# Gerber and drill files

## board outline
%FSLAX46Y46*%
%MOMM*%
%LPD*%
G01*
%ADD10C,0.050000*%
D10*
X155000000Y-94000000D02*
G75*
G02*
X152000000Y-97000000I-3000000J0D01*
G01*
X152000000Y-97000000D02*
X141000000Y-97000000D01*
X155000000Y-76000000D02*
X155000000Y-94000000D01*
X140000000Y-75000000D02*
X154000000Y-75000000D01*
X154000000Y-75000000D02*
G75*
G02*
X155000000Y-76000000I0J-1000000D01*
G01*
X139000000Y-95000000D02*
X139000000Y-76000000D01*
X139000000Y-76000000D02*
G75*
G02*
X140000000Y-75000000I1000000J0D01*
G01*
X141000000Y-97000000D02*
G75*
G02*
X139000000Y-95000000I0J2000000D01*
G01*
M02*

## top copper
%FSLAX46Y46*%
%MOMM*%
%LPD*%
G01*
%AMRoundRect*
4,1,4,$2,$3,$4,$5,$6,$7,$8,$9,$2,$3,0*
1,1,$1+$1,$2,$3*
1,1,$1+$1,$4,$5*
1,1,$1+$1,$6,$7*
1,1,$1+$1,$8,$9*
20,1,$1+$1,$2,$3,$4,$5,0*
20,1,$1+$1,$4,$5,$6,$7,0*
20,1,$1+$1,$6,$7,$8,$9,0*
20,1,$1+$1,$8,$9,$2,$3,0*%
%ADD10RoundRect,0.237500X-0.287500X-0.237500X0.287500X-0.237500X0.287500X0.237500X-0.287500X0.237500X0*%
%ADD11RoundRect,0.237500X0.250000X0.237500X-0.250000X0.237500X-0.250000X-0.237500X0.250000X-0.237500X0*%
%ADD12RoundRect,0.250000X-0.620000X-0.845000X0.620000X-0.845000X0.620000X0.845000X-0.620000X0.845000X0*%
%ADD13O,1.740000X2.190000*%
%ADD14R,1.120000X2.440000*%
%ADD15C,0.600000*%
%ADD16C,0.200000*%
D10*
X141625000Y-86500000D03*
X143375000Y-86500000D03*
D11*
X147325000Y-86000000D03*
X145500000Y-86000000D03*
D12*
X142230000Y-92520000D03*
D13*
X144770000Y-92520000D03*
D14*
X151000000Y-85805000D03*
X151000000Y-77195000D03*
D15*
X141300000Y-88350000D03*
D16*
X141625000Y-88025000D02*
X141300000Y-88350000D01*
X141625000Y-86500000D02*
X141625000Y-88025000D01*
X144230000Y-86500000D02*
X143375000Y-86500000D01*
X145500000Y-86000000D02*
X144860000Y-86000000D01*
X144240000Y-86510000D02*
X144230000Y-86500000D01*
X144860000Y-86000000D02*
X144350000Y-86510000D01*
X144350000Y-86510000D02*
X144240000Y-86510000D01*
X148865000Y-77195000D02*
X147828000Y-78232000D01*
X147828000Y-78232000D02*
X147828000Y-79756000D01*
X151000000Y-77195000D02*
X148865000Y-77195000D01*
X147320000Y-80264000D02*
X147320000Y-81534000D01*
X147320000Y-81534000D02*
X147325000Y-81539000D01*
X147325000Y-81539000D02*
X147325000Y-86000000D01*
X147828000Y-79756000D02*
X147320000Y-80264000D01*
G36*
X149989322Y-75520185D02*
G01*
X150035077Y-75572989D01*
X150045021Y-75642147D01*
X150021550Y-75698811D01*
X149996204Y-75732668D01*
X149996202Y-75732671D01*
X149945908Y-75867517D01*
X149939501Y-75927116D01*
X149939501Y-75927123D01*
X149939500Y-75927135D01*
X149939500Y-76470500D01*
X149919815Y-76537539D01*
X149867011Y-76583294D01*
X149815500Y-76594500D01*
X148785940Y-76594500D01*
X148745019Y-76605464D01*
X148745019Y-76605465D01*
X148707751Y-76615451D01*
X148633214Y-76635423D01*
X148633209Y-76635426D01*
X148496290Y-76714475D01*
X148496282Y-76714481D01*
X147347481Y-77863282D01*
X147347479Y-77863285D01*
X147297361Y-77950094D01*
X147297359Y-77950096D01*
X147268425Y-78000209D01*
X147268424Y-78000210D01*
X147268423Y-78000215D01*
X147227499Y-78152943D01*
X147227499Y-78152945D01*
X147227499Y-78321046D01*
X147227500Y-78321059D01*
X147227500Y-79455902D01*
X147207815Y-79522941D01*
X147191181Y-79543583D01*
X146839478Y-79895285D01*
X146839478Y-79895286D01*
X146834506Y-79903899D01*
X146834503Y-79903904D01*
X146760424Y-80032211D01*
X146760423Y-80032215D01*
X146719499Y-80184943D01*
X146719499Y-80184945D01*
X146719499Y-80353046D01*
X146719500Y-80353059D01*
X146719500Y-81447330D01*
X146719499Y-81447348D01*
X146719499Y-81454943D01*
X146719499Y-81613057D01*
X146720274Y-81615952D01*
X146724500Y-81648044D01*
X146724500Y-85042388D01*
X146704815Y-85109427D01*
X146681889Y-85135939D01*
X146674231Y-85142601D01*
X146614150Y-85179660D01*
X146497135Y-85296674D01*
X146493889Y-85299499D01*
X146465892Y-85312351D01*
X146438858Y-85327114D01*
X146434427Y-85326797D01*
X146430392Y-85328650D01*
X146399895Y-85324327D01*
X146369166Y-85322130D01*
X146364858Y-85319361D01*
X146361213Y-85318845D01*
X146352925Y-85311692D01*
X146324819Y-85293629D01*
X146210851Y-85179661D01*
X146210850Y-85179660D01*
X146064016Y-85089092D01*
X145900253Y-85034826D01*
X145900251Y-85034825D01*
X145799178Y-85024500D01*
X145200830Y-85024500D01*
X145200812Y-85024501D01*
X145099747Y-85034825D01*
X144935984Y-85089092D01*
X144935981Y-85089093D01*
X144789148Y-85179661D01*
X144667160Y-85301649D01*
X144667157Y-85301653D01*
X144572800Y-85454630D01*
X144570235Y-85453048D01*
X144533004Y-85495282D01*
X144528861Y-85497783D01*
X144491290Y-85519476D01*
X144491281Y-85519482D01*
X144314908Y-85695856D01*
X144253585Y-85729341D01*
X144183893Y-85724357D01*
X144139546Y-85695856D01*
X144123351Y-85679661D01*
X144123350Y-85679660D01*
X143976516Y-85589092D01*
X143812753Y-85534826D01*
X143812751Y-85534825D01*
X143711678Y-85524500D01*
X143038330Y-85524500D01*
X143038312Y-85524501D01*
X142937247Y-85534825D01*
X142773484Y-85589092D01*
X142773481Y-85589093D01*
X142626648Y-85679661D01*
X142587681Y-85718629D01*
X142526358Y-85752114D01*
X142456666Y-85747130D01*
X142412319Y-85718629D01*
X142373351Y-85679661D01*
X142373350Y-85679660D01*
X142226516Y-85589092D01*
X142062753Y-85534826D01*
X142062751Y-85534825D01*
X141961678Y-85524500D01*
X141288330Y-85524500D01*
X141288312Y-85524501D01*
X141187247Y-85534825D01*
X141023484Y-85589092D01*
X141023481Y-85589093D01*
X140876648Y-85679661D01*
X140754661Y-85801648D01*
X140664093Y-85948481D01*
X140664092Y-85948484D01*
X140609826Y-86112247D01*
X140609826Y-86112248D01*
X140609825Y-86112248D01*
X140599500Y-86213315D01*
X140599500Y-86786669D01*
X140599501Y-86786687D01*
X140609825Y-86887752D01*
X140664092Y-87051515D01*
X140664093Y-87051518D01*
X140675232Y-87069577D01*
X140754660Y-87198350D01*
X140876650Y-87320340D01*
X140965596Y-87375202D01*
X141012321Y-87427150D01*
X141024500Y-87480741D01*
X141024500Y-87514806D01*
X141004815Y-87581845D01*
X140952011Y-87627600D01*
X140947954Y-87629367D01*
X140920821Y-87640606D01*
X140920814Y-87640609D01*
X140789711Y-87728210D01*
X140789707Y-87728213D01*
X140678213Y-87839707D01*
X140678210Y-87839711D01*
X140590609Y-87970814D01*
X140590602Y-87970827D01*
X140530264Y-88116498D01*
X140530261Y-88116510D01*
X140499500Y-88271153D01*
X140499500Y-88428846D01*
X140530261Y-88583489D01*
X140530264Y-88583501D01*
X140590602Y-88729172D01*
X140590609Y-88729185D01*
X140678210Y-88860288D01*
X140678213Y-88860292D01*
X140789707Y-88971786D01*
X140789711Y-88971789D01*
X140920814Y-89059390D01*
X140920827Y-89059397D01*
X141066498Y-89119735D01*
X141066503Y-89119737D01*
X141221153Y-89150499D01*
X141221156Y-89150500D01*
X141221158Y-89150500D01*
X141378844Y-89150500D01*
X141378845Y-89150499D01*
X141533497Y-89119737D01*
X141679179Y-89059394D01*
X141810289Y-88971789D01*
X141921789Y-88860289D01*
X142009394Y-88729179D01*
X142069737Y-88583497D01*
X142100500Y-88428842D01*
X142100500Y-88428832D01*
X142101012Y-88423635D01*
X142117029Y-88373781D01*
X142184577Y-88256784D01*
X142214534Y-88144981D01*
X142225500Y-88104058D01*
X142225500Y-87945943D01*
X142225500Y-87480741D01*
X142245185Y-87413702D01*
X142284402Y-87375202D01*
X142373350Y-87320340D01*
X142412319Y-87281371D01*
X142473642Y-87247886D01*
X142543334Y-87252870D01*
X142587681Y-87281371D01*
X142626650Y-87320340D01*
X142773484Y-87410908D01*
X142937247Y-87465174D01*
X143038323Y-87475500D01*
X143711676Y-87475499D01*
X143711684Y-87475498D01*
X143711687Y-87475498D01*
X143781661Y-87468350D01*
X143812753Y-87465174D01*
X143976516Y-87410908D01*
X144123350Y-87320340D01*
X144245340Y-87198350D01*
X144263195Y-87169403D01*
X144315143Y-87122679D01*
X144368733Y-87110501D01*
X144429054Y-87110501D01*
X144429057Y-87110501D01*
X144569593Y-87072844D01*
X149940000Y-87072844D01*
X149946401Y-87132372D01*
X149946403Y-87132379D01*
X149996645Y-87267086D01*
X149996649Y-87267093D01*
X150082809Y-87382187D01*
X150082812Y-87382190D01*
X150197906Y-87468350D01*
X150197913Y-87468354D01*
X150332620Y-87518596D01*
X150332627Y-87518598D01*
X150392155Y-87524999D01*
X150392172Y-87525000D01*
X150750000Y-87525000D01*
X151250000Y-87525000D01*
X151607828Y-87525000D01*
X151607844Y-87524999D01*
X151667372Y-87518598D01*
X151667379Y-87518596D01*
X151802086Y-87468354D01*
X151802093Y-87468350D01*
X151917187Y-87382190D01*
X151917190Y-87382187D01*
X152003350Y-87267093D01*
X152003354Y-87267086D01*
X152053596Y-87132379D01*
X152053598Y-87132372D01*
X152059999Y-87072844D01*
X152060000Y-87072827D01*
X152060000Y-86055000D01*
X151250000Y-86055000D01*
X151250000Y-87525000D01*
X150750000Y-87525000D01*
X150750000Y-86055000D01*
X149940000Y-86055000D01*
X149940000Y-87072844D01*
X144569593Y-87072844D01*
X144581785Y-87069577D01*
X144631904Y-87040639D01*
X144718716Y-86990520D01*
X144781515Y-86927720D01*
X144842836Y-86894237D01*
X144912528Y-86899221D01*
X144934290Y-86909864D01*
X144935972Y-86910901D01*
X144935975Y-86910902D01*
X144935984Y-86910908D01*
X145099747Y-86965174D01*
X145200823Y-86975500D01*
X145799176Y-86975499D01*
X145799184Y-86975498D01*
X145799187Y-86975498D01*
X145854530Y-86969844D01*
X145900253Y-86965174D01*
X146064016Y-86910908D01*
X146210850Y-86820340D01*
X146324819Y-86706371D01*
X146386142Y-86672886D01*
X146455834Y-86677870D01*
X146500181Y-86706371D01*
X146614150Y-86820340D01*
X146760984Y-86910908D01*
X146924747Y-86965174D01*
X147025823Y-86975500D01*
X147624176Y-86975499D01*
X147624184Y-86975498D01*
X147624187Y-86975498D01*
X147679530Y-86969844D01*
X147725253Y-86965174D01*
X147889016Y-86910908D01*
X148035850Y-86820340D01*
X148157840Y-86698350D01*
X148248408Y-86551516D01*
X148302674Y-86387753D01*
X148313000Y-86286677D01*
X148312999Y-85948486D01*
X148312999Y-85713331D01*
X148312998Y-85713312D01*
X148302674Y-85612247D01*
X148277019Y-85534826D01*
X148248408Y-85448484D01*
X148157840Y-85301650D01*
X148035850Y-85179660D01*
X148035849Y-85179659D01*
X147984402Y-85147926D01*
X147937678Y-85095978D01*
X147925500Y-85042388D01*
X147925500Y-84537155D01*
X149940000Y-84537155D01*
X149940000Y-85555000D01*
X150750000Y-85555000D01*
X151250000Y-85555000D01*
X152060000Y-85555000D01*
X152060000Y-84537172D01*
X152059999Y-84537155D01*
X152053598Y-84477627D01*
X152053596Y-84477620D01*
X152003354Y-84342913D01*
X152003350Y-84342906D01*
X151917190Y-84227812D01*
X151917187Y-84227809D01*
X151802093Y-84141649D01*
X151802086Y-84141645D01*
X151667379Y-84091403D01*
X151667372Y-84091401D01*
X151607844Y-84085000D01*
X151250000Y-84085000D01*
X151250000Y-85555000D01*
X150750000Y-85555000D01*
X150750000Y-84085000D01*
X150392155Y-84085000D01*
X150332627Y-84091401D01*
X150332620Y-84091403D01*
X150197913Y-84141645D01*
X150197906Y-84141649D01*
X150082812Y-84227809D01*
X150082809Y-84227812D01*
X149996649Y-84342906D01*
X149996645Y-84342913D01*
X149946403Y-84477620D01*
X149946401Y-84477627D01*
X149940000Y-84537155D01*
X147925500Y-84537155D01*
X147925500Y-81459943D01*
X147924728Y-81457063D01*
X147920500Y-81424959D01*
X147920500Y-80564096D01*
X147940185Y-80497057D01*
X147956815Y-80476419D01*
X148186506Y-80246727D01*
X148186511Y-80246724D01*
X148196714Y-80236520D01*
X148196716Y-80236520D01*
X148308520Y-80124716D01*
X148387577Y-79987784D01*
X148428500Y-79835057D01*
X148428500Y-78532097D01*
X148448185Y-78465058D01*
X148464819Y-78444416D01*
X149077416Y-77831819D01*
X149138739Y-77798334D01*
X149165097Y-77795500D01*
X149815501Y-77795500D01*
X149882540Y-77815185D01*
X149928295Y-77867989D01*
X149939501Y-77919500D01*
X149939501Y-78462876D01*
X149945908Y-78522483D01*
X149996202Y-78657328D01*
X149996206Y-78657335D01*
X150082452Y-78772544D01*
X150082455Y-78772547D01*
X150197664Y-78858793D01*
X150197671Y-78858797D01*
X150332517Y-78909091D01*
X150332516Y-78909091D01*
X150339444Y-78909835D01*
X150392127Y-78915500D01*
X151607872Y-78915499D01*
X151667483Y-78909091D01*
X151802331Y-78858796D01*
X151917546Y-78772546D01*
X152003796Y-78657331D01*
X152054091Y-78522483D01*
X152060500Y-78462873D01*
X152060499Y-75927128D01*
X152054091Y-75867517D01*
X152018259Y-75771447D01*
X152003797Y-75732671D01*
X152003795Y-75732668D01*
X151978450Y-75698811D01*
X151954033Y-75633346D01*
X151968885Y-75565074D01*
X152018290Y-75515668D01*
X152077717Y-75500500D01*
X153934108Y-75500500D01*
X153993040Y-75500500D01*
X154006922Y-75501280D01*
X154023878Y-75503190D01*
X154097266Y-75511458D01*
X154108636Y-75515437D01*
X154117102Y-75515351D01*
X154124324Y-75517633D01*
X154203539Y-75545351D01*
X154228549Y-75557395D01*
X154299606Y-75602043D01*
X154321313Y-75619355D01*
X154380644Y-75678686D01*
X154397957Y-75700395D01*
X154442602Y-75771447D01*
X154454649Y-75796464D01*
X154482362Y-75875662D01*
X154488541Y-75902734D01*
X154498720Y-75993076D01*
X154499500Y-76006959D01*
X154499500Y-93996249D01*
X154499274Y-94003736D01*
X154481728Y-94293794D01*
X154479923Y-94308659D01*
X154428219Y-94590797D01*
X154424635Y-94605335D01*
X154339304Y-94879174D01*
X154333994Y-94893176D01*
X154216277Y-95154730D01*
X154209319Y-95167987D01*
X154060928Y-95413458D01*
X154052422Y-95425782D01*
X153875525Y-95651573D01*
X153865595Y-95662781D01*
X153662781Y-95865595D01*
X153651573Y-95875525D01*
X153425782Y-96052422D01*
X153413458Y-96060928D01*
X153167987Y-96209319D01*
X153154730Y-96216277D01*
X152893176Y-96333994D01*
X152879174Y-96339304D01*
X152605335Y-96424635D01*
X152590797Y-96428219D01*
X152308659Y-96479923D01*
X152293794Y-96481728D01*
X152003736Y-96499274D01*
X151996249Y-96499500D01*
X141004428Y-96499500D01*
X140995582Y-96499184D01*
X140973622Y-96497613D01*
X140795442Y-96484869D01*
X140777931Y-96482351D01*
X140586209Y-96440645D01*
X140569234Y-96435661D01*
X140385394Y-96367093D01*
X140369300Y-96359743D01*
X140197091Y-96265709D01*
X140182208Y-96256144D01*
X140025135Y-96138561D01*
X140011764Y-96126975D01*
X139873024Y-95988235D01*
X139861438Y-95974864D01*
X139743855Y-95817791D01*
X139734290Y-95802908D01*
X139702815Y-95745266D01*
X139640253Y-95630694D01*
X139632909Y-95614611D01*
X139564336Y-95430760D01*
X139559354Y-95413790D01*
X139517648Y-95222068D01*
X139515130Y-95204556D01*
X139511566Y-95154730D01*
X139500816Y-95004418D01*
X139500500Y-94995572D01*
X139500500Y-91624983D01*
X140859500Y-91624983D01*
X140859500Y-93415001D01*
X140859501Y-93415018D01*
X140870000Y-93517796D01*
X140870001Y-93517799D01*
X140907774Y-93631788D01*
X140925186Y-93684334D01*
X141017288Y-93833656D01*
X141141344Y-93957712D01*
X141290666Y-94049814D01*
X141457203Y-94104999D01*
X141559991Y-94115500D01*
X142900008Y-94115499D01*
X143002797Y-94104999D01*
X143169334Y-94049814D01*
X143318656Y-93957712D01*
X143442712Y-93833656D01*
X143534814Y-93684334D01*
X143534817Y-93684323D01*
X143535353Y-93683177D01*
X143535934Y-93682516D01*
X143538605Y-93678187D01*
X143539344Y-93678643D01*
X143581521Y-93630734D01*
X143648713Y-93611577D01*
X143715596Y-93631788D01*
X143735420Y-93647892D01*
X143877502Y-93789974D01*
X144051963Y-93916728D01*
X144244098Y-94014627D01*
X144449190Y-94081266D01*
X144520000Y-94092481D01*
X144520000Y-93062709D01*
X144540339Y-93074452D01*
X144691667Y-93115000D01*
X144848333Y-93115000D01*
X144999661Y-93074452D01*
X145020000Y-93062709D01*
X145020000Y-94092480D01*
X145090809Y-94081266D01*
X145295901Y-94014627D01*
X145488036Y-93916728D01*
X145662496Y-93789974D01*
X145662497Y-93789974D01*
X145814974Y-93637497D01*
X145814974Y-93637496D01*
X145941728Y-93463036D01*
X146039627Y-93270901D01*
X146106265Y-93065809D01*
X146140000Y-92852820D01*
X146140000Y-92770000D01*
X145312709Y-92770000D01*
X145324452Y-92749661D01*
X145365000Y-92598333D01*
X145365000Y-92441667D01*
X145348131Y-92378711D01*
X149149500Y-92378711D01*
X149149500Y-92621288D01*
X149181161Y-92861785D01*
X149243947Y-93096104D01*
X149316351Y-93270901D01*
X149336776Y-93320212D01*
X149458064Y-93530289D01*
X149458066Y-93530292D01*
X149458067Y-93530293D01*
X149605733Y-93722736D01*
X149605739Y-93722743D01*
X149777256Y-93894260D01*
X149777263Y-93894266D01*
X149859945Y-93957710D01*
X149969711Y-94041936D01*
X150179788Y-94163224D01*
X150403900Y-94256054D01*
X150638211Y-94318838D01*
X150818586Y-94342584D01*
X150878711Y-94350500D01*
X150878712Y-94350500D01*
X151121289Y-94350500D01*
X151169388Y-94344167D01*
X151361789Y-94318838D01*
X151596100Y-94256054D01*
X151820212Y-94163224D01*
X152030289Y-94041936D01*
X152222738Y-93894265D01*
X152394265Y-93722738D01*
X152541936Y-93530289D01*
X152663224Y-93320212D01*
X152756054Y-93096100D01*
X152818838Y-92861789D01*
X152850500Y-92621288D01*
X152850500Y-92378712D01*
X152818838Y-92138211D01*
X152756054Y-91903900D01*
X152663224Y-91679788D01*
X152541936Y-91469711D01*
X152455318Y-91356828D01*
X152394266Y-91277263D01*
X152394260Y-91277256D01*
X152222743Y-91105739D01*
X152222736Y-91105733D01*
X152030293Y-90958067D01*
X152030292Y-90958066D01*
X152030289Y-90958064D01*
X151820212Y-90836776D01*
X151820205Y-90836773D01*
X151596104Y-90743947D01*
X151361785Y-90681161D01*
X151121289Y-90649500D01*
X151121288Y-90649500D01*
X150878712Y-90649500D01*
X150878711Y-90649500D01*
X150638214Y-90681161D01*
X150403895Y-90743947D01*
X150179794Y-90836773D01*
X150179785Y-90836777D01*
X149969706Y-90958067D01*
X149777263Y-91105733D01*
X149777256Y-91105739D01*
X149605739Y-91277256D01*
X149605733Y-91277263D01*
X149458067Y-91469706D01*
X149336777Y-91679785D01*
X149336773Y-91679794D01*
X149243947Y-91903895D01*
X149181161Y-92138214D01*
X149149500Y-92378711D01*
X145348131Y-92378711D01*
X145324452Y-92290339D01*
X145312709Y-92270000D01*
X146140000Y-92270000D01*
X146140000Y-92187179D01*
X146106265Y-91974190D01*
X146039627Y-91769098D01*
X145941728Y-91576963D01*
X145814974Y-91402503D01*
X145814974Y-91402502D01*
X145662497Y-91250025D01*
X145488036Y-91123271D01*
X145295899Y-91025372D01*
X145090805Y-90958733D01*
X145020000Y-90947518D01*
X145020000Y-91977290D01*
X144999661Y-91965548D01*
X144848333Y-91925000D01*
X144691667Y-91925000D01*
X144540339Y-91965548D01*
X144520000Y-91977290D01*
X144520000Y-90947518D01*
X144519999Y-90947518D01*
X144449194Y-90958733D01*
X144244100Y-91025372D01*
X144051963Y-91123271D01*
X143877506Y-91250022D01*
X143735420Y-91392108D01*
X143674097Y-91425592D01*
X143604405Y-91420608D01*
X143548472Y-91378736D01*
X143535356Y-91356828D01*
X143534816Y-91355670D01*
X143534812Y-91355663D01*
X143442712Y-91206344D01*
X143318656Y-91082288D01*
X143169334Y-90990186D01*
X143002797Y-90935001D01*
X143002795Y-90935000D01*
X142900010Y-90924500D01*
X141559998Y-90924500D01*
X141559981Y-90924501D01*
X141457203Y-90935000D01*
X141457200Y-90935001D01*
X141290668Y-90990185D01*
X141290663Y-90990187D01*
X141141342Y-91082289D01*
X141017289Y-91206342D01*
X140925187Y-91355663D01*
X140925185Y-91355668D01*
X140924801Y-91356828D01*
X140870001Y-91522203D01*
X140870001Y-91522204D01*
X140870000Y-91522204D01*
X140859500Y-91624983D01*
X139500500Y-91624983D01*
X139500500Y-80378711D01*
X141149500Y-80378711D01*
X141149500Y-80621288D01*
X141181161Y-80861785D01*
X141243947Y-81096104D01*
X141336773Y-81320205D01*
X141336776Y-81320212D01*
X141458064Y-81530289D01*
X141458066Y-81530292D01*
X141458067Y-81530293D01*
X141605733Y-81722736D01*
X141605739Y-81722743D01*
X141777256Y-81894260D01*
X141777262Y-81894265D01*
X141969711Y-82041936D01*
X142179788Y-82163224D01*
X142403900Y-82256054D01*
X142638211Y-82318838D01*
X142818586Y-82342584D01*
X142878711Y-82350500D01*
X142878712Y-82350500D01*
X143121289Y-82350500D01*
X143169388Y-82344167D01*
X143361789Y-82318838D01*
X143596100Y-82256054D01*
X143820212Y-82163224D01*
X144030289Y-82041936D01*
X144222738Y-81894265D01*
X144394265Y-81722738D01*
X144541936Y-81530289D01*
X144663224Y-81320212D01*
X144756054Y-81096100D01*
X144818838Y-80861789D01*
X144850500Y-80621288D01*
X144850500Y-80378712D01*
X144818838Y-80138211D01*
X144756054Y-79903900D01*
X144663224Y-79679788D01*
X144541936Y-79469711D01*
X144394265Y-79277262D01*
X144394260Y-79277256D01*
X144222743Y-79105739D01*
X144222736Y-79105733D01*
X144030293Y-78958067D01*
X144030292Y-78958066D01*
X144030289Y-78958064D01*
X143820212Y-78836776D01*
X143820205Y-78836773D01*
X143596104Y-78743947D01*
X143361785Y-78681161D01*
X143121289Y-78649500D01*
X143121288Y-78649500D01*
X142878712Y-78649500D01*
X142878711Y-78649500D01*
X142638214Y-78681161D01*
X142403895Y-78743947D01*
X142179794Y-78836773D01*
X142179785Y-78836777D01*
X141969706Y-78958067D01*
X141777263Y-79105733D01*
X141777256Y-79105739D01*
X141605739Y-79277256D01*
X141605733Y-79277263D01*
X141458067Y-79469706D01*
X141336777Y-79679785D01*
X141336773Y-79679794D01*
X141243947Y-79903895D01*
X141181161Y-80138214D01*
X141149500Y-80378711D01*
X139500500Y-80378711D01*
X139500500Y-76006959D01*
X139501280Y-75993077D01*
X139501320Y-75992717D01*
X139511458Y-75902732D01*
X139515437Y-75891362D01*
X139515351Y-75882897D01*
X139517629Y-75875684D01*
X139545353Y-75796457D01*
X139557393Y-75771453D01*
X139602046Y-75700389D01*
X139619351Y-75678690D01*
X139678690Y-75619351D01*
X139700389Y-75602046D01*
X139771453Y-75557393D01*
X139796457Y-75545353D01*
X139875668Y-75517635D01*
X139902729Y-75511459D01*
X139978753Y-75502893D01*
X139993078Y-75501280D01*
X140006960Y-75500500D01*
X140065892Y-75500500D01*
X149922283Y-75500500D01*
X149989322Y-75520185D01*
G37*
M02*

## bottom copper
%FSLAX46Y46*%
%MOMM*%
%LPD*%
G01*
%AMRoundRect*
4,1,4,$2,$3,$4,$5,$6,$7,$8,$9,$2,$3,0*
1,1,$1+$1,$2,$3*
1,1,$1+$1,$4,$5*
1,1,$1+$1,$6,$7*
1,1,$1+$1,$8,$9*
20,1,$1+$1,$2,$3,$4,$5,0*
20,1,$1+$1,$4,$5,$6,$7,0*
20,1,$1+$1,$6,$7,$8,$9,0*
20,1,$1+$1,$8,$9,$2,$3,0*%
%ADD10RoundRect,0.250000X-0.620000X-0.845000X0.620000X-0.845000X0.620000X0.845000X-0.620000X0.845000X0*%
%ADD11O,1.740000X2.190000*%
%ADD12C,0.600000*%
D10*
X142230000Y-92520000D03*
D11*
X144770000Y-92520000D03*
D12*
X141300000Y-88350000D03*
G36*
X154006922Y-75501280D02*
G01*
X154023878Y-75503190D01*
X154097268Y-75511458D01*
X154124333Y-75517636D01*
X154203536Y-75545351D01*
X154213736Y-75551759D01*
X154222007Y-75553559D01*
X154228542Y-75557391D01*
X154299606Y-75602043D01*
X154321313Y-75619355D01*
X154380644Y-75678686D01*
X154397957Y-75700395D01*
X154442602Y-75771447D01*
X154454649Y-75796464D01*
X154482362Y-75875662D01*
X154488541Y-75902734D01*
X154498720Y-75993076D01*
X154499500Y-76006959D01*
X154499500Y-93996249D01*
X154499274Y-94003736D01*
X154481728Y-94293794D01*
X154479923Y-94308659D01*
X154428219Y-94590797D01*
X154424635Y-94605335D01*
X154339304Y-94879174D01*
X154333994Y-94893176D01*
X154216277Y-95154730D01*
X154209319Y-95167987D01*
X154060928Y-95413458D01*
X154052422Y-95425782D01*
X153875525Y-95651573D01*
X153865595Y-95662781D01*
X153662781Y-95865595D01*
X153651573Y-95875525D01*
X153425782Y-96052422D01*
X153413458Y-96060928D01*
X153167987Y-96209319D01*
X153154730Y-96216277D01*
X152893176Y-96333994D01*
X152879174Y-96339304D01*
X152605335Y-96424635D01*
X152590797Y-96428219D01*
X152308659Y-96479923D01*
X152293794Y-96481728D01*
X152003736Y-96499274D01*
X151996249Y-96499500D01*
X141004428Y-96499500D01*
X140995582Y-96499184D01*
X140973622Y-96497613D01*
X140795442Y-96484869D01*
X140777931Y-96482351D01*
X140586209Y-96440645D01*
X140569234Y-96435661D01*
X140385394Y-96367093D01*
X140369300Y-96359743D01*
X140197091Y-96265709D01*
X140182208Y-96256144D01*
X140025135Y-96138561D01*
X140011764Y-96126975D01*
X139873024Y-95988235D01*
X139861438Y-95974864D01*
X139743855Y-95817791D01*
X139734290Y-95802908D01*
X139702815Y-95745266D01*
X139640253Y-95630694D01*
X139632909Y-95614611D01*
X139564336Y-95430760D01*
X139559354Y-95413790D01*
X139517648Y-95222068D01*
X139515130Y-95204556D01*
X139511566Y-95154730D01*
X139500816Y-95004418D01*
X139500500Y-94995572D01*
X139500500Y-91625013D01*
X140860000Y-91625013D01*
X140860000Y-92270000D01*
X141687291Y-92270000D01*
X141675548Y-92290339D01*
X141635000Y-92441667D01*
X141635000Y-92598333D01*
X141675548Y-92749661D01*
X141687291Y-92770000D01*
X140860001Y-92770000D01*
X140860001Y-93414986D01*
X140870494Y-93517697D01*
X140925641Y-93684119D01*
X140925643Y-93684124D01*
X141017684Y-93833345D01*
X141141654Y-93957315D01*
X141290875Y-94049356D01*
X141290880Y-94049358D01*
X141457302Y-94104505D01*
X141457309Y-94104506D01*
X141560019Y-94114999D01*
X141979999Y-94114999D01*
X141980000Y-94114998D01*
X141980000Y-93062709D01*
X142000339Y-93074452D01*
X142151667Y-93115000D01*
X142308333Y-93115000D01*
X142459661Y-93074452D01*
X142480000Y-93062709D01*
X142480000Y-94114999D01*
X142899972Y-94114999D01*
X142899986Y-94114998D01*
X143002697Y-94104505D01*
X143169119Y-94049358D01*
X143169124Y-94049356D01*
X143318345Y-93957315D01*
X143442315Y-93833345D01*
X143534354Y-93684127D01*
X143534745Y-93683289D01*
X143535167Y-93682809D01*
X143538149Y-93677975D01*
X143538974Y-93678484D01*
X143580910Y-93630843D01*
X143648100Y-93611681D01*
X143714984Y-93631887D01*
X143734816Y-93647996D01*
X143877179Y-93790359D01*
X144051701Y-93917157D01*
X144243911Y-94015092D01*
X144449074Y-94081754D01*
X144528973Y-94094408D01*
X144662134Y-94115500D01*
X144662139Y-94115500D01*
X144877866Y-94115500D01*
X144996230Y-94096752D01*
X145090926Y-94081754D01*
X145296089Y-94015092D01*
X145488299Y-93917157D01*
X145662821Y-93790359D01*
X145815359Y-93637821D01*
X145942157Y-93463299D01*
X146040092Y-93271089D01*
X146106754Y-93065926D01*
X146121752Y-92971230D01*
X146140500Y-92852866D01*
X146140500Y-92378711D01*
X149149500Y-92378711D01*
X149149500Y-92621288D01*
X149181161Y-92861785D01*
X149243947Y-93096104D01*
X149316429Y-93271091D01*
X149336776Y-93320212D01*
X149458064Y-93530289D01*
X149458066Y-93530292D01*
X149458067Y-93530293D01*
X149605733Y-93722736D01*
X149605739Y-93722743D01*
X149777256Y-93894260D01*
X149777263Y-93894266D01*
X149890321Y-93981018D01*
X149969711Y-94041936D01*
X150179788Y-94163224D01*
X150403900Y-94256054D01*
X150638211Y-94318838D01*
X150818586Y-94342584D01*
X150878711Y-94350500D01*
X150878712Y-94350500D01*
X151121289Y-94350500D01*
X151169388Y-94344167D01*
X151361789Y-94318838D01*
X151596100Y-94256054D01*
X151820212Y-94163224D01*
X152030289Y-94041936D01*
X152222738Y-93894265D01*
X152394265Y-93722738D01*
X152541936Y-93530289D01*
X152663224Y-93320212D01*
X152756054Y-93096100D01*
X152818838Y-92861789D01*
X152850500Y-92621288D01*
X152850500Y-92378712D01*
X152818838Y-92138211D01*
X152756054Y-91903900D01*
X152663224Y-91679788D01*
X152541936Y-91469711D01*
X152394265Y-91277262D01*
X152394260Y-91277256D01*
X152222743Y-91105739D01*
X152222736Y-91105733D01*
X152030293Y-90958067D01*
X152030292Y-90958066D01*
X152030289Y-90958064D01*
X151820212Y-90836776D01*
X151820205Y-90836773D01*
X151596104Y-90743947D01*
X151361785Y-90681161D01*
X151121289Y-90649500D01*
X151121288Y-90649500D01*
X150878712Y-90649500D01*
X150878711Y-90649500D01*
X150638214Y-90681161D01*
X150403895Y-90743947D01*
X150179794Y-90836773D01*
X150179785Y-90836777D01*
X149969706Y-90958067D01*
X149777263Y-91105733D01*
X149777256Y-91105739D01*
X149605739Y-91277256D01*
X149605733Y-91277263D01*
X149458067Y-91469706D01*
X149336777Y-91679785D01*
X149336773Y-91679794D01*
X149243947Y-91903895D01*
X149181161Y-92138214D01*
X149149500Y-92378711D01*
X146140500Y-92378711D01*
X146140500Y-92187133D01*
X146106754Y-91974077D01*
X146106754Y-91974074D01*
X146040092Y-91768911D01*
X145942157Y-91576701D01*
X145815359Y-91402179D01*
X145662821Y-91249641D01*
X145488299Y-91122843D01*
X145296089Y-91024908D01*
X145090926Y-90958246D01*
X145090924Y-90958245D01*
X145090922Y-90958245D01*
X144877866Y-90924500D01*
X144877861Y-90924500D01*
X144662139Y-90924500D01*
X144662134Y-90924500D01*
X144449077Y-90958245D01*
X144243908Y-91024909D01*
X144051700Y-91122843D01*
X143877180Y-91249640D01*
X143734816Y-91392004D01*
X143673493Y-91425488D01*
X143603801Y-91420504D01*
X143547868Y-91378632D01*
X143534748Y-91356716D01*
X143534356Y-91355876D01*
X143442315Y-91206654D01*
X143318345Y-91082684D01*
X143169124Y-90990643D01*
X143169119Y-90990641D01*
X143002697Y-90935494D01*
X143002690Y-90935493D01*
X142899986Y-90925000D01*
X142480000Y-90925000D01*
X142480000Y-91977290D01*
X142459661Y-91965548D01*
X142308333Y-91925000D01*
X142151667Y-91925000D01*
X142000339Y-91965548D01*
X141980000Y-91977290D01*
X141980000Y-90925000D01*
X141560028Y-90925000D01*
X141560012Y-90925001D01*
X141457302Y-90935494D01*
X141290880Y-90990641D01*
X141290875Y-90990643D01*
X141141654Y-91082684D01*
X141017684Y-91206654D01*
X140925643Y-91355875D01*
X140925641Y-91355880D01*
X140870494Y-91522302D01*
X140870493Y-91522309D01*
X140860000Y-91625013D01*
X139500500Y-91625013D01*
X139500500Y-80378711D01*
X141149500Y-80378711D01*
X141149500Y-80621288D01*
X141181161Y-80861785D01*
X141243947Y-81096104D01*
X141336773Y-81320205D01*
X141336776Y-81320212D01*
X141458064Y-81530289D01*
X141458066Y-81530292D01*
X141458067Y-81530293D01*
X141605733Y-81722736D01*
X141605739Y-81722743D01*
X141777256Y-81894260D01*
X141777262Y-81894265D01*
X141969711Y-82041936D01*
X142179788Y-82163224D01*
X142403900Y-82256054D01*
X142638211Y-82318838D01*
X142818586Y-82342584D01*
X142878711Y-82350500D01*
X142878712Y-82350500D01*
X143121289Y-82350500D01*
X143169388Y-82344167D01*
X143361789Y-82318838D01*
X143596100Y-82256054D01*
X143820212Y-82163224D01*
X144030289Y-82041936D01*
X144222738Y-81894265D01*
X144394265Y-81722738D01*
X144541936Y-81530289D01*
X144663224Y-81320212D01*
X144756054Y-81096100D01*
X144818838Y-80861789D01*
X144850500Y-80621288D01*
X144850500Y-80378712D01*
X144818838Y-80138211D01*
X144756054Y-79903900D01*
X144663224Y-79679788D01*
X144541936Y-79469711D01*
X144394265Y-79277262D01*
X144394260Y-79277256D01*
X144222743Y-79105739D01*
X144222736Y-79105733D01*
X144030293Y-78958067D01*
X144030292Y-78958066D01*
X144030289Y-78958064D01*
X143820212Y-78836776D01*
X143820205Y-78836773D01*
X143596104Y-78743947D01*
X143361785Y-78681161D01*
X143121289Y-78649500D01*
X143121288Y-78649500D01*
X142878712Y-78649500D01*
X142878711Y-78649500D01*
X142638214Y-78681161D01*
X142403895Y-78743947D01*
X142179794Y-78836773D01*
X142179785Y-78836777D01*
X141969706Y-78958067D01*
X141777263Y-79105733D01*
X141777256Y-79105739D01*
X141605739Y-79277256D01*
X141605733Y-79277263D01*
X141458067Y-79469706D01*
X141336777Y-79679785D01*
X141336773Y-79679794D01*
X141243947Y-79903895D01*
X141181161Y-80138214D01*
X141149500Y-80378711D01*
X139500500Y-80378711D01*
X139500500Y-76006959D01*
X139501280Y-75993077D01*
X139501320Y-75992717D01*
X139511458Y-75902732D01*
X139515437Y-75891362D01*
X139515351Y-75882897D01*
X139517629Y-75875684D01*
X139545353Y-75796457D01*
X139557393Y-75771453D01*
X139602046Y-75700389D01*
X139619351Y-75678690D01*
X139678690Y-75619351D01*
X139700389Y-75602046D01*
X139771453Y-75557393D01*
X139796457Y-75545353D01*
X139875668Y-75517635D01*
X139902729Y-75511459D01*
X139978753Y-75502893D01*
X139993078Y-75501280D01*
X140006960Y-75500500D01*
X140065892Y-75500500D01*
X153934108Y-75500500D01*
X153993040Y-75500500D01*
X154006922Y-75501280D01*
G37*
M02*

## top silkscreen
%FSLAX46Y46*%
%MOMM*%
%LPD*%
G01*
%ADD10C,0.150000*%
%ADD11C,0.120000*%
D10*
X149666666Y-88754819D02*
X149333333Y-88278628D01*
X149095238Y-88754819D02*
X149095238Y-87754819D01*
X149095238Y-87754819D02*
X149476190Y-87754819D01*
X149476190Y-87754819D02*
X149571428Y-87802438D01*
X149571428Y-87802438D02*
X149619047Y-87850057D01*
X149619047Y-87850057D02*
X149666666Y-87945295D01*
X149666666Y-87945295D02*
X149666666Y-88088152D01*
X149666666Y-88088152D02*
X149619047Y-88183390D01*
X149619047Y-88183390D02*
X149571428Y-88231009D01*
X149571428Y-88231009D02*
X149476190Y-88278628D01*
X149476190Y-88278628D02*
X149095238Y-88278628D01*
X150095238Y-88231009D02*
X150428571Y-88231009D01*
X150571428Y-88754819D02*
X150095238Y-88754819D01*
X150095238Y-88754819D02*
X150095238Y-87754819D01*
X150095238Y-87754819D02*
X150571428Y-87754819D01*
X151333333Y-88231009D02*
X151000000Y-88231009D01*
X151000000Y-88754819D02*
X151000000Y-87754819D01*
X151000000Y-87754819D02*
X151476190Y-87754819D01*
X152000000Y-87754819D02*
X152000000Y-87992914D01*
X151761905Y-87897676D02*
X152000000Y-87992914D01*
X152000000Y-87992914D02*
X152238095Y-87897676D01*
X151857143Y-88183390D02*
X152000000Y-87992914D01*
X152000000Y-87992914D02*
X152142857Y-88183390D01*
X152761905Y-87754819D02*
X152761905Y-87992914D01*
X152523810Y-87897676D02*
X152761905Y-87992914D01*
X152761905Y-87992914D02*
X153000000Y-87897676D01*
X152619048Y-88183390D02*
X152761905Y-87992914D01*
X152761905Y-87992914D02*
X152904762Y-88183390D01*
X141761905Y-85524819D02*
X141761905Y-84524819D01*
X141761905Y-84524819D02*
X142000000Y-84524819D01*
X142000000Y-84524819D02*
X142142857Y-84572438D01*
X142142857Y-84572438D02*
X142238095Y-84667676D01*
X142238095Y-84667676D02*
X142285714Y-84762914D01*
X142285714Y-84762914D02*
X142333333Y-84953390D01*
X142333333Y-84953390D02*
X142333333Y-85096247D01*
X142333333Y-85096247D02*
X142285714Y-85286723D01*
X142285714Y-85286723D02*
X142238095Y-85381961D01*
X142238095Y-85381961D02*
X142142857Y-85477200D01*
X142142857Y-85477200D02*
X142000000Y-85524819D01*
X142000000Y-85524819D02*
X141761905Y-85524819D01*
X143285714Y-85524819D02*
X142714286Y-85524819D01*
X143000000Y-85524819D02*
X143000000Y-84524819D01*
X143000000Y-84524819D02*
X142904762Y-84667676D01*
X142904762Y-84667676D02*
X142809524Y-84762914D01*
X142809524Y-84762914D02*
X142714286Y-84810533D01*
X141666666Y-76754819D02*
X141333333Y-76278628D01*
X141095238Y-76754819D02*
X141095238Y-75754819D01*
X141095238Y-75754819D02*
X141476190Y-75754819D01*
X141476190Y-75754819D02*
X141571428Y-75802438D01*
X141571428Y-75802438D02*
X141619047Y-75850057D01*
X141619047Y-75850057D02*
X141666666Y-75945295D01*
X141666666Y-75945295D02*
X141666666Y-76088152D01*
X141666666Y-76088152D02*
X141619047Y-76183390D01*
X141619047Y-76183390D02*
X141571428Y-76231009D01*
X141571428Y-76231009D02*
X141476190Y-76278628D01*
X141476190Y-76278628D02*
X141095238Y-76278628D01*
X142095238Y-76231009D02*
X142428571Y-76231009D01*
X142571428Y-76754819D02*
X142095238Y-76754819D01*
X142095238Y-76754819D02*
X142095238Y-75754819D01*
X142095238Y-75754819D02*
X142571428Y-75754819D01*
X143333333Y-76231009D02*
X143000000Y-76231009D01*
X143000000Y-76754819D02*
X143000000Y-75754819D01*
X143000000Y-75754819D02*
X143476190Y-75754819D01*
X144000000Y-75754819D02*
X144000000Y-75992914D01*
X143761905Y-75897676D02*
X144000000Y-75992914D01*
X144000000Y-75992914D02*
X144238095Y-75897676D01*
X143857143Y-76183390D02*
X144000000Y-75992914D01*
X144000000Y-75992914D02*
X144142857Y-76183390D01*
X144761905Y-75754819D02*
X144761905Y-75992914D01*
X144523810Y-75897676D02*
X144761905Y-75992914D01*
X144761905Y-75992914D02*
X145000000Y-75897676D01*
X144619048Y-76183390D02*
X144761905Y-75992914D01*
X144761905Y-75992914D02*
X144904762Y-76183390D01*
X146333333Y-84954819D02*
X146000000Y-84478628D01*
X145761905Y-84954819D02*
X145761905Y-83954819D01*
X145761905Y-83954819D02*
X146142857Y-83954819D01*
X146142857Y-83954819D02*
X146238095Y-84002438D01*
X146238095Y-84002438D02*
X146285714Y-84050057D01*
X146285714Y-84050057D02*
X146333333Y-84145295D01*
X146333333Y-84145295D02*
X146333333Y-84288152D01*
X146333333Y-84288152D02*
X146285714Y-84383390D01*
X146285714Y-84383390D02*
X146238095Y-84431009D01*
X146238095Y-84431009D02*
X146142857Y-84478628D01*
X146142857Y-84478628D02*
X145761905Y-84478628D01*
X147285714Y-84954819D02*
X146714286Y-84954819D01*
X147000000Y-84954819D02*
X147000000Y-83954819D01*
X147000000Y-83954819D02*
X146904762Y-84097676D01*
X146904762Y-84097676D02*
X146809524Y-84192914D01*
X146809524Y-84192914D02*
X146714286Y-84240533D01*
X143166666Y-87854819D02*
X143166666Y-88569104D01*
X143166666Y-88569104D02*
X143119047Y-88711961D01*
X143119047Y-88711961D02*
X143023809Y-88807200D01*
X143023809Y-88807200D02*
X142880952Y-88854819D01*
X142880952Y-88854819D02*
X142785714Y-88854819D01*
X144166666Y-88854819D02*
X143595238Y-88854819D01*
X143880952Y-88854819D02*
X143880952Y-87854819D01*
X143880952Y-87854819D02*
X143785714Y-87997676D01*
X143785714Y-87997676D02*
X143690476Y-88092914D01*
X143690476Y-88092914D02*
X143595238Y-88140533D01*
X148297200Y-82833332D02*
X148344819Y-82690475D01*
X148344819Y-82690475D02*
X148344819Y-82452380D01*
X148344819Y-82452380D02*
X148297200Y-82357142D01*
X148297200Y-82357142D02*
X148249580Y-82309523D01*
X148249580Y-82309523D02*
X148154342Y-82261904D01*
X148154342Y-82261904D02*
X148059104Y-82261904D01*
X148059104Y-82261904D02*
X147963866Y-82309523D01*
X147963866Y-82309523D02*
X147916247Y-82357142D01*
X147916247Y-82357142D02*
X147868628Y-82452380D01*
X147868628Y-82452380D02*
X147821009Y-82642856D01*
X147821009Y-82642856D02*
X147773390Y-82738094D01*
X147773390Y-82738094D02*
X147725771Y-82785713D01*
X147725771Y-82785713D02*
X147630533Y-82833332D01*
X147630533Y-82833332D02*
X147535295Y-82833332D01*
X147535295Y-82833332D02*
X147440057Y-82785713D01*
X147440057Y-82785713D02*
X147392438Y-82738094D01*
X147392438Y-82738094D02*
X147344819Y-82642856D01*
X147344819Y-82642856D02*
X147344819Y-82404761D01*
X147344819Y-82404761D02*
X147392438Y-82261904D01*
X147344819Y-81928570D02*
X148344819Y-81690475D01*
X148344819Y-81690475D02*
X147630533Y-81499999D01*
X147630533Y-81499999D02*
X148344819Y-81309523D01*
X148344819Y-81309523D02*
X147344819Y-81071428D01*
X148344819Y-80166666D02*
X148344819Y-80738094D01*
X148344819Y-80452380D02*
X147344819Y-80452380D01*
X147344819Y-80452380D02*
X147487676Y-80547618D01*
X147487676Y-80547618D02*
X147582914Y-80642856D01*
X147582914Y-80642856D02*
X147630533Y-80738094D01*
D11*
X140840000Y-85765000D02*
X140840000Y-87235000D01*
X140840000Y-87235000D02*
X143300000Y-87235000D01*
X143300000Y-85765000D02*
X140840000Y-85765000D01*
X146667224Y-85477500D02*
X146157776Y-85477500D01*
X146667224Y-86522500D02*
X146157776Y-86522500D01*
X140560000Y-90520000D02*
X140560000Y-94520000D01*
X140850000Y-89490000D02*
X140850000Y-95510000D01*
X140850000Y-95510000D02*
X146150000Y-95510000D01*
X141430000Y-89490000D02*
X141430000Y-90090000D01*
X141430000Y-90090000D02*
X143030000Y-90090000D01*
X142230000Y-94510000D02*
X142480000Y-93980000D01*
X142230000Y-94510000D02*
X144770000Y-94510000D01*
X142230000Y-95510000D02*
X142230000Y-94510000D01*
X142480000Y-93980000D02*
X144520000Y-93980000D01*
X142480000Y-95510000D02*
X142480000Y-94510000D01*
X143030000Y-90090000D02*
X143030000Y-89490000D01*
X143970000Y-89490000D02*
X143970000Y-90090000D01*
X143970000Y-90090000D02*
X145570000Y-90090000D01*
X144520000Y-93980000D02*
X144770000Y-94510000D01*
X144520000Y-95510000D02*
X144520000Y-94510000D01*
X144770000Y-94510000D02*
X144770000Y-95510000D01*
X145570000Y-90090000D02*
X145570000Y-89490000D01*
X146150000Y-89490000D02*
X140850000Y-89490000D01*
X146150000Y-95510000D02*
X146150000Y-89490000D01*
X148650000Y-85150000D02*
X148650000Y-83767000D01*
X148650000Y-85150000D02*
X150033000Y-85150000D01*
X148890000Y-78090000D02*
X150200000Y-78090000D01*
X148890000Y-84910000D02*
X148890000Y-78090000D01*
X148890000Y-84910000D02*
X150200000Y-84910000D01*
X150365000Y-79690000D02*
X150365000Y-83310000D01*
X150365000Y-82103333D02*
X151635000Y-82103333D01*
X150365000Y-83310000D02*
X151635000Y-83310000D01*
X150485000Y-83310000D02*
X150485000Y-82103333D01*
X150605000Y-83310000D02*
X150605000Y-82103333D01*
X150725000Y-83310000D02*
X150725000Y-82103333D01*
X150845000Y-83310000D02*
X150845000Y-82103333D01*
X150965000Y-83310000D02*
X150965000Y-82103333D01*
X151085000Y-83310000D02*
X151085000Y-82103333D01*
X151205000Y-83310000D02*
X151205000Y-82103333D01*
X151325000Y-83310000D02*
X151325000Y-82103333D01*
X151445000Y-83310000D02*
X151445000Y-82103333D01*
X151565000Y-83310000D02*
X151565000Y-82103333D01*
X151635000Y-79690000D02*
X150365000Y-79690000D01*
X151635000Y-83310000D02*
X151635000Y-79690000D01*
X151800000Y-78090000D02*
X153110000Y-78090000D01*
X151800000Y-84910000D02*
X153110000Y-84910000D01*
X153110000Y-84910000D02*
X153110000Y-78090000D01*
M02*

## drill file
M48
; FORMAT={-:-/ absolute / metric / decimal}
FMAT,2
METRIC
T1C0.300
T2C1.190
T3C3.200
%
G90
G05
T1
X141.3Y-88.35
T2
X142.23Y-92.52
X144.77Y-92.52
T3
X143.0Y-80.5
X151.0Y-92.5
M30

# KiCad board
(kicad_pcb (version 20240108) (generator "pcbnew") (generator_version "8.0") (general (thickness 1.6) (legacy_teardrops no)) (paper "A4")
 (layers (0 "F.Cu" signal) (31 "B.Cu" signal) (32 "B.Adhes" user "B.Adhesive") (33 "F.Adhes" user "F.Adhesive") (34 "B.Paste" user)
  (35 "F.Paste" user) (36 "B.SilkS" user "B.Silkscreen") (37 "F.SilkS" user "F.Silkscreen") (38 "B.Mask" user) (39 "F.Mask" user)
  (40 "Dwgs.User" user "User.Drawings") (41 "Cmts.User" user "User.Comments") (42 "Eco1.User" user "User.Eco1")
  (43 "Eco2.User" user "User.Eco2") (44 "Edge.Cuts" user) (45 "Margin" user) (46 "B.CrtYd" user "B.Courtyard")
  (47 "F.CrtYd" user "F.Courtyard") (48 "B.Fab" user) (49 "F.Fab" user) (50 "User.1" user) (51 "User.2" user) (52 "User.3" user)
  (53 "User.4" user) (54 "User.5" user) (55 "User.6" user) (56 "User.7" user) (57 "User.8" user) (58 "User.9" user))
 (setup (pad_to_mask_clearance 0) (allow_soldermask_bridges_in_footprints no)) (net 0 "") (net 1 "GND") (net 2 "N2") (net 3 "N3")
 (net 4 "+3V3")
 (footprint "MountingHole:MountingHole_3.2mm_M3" (layer "F.Cu") (at 151 92.5)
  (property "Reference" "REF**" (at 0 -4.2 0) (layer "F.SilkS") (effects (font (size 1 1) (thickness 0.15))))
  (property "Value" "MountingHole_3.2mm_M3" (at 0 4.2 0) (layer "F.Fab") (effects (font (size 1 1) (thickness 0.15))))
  (pad "" np_thru_hole circle (at 0 0) (size 3.2 3.2) (drill 3.2) (layers "*.Cu" "*.Mask")))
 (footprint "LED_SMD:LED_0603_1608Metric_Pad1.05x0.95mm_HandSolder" (layer "F.Cu") (at 142.5 86.5)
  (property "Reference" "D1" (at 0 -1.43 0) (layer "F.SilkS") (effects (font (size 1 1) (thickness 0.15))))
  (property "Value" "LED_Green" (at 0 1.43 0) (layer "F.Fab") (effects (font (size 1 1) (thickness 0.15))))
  (fp_line (start -1.66 -0.735) (end -1.66 0.735) (stroke (width 0.12) (type solid)) (layer "F.SilkS"))
  (fp_line (start -1.66 0.735) (end 0.8 0.735) (stroke (width 0.12) (type solid)) (layer "F.SilkS"))
  (fp_line (start 0.8 -0.735) (end -1.66 -0.735) (stroke (width 0.12) (type solid)) (layer "F.SilkS"))
  (pad "1" smd roundrect (at -0.875 0) (size 1.05 0.95) (layers "F.Cu" "F.Paste" "F.Mask") (roundrect_rratio 0.25) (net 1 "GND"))
  (pad "2" smd roundrect (at 0.875 0) (size 1.05 0.95) (layers "F.Cu" "F.Paste" "F.Mask") (roundrect_rratio 0.25) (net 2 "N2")))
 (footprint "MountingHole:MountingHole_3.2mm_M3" (layer "F.Cu") (at 143 80.5)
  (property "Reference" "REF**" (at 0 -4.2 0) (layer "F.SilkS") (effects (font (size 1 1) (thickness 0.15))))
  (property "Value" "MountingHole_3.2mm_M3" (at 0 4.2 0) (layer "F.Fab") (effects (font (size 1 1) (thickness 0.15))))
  (pad "" np_thru_hole circle (at 0 0) (size 3.2 3.2) (drill 3.2) (layers "*.Cu" "*.Mask")))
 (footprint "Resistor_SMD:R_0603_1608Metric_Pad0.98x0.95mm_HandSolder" (layer "F.Cu") (at 146.4125 86 180)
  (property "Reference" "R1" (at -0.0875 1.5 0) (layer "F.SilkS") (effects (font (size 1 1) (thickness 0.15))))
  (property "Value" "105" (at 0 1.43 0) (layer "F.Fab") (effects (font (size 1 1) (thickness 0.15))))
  (fp_line (start -0.254724 0.5225) (end 0.254724 0.5225) (stroke (width 0.12) (type solid)) (layer "F.SilkS"))
  (fp_line (start -0.254724 -0.5225) (end 0.254724 -0.5225) (stroke (width 0.12) (type solid)) (layer "F.SilkS"))
  (pad "1" smd roundrect (at -0.9125 0 180) (size 0.975 0.95) (layers "F.Cu" "F.Paste" "F.Mask") (roundrect_rratio 0.25) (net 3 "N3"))
  (pad "2" smd roundrect (at 0.9125 0 180) (size 0.975 0.95) (layers "F.Cu" "F.Paste" "F.Mask") (roundrect_rratio 0.25) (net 2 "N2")))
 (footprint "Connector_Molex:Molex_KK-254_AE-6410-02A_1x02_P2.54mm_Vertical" (layer "F.Cu") (at 142.23 92.52)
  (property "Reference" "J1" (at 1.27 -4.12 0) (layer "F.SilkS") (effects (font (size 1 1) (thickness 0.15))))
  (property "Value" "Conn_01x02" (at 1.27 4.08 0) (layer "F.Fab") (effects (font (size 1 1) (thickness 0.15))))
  (fp_line (start -1.67 -2) (end -1.67 2) (stroke (width 0.12) (type solid)) (layer "F.SilkS"))
  (fp_line (start -1.38 -3.03) (end -1.38 2.99) (stroke (width 0.12) (type solid)) (layer "F.SilkS"))
  (fp_line (start -1.38 2.99) (end 3.92 2.99) (stroke (width 0.12) (type solid)) (layer "F.SilkS"))
  (fp_line (start -0.8 -3.03) (end -0.8 -2.43) (stroke (width 0.12) (type solid)) (layer "F.SilkS"))
  (fp_line (start -0.8 -2.43) (end 0.8 -2.43) (stroke (width 0.12) (type solid)) (layer "F.SilkS"))
  (fp_line (start 0 1.99) (end 0.25 1.46) (stroke (width 0.12) (type solid)) (layer "F.SilkS"))
  (fp_line (start 0 1.99) (end 2.54 1.99) (stroke (width 0.12) (type solid)) (layer "F.SilkS"))
  (fp_line (start 0 2.99) (end 0 1.99) (stroke (width 0.12) (type solid)) (layer "F.SilkS"))
  (fp_line (start 0.25 1.46) (end 2.29 1.46) (stroke (width 0.12) (type solid)) (layer "F.SilkS"))
  (fp_line (start 0.25 2.99) (end 0.25 1.99) (stroke (width 0.12) (type solid)) (layer "F.SilkS"))
  (fp_line (start 0.8 -2.43) (end 0.8 -3.03) (stroke (width 0.12) (type solid)) (layer "F.SilkS"))
  (fp_line (start 1.74 -3.03) (end 1.74 -2.43) (stroke (width 0.12) (type solid)) (layer "F.SilkS"))
  (fp_line (start 1.74 -2.43) (end 3.34 -2.43) (stroke (width 0.12) (type solid)) (layer "F.SilkS"))
  (fp_line (start 2.29 1.46) (end 2.54 1.99) (stroke (width 0.12) (type solid)) (layer "F.SilkS"))
  (fp_line (start 2.29 2.99) (end 2.29 1.99) (stroke (width 0.12) (type solid)) (layer "F.SilkS"))
  (fp_line (start 2.54 1.99) (end 2.54 2.99) (stroke (width 0.12) (type solid)) (layer "F.SilkS"))
  (fp_line (start 3.34 -2.43) (end 3.34 -3.03) (stroke (width 0.12) (type solid)) (layer "F.SilkS"))
  (fp_line (start 3.92 -3.03) (end -1.38 -3.03) (stroke (width 0.12) (type solid)) (layer "F.SilkS"))
  (fp_line (start 3.92 2.99) (end 3.92 -3.03) (stroke (width 0.12) (type solid)) (layer "F.SilkS"))
  (pad "1" thru_hole roundrect (at 0 0) (size 1.74 2.19) (drill 1.19) (layers "*.Cu" "*.Mask") (remove_unused_layers no)
   (roundrect_rratio 0.143678) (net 1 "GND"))
  (pad "2" thru_hole oval (at 2.54 0) (size 1.74 2.19) (drill 1.19) (layers "*.Cu" "*.Mask") (remove_unused_layers no) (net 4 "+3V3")))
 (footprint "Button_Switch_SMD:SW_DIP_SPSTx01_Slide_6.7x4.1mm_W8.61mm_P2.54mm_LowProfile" (layer "F.Cu") (at 151 81.5 90)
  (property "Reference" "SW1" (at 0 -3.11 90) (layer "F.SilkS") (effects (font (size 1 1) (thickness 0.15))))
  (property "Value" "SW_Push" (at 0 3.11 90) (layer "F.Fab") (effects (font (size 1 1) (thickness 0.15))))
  (fp_line (start -3.65 -2.35) (end -2.267 -2.35) (stroke (width 0.12) (type solid)) (layer "F.SilkS"))
  (fp_line (start -3.65 -2.35) (end -3.65 -0.967) (stroke (width 0.12) (type solid)) (layer "F.SilkS"))
  (fp_line (start 3.41 -2.11) (end 3.41 -0.8) (stroke (width 0.12) (type solid)) (layer "F.SilkS"))
  (fp_line (start -3.41 -2.11) (end 3.41 -2.11) (stroke (width 0.12) (type solid)) (layer "F.SilkS"))
  (fp_line (start -3.41 -2.11) (end -3.41 -0.8) (stroke (width 0.12) (type solid)) (layer "F.SilkS"))
  (fp_line (start 1.81 -0.635) (end -1.81 -0.635) (stroke (width 0.12) (type solid)) (layer "F.SilkS"))
  (fp_line (start -0.603333 -0.635) (end -0.603333 0.635) (stroke (width 0.12) (type solid)) (layer "F.SilkS"))
  (fp_line (start -1.81 -0.635) (end -1.81 0.635) (stroke (width 0.12) (type solid)) (layer "F.SilkS"))
  (fp_line (start -1.81 -0.515) (end -0.603333 -0.515) (stroke (width 0.12) (type solid)) (layer "F.SilkS"))
  (fp_line (start -1.81 -0.395) (end -0.603333 -0.395) (stroke (width 0.12) (type solid)) (layer "F.SilkS"))
  (fp_line (start -1.81 -0.275) (end -0.603333 -0.275) (stroke (width 0.12) (type solid)) (layer "F.SilkS"))
  (fp_line (start -1.81 -0.155) (end -0.603333 -0.155) (stroke (width 0.12) (type solid)) (layer "F.SilkS"))
  (fp_line (start -1.81 -0.035) (end -0.603333 -0.035) (stroke (width 0.12) (type solid)) (layer "F.SilkS"))
  (fp_line (start -1.81 0.085) (end -0.603333 0.085) (stroke (width 0.12) (type solid)) (layer "F.SilkS"))
  (fp_line (start -1.81 0.205) (end -0.603333 0.205) (stroke (width 0.12) (type solid)) (layer "F.SilkS"))
  (fp_line (start -1.81 0.325) (end -0.603333 0.325) (stroke (width 0.12) (type solid)) (layer "F.SilkS"))
  (fp_line (start -1.81 0.445) (end -0.603333 0.445) (stroke (width 0.12) (type solid)) (layer "F.SilkS"))
  (fp_line (start -1.81 0.565) (end -0.603333 0.565) (stroke (width 0.12) (type solid)) (layer "F.SilkS"))
  (fp_line (start 1.81 0.635) (end 1.81 -0.635) (stroke (width 0.12) (type solid)) (layer "F.SilkS"))
  (fp_line (start -1.81 0.635) (end 1.81 0.635) (stroke (width 0.12) (type solid)) (layer "F.SilkS"))
  (fp_line (start 3.41 0.8) (end 3.41 2.11) (stroke (width 0.12) (type solid)) (layer "F.SilkS"))
  (fp_line (start -3.41 0.8) (end -3.41 2.11) (stroke (width 0.12) (type solid)) (layer "F.SilkS"))
  (fp_line (start -3.41 2.11) (end 3.41 2.11) (stroke (width 0.12) (type solid)) (layer "F.SilkS"))
  (pad "1" smd rect (at -4.305 0 90) (size 2.44 1.12) (layers "F.Cu" "F.Paste" "F.Mask") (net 4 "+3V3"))
  (pad "2" smd rect (at 4.305 0 90) (size 2.44 1.12) (layers "F.Cu" "F.Paste" "F.Mask") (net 3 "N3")))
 (gr_arc (start 155 94) (mid 154.12132 96.12132) (end 152 97) (stroke (width 0.05) (type default)) (layer "Edge.Cuts"))
 (gr_line (start 152 97) (end 141 97) (stroke (width 0.05) (type default)) (layer "Edge.Cuts"))
 (gr_line (start 155 76) (end 155 94) (stroke (width 0.05) (type default)) (layer "Edge.Cuts"))
 (gr_line (start 140 75) (end 154 75) (stroke (width 0.05) (type default)) (layer "Edge.Cuts"))
 (gr_arc (start 154 75) (mid 154.707107 75.292893) (end 155 76) (stroke (width 0.05) (type default)) (layer "Edge.Cuts"))
 (gr_line (start 139 95) (end 139 76) (stroke (width 0.05) (type default)) (layer "Edge.Cuts"))
 (gr_arc (start 139 76) (mid 139.292893 75.292893) (end 140 75) (stroke (width 0.05) (type default)) (layer "Edge.Cuts"))
 (gr_arc (start 141 97) (mid 139.585786 96.414214) (end 139 95) (stroke (width 0.05) (type default)) (layer "Edge.Cuts"))
 (segment (start 141.625 88.025) (end 141.3 88.35) (width 0.2) (layer "F.Cu") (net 1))
 (segment (start 141.625 86.5) (end 141.625 88.025) (width 0.2) (layer "F.Cu") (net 1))
 (via (at 141.3 88.35) (size 0.6) (drill 0.3) (layers "F.Cu" "B.Cu") (free yes) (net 1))
 (segment (start 144.23 86.5) (end 143.375 86.5) (width 0.2) (layer "F.Cu") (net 2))
 (segment (start 145.5 86) (end 144.86 86) (width 0.2) (layer "F.Cu") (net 2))
 (segment (start 144.24 86.51) (end 144.23 86.5) (width 0.2) (layer "F.Cu") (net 2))
 (segment (start 144.86 86) (end 144.35 86.51) (width 0.2) (layer "F.Cu") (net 2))
 (segment (start 144.35 86.51) (end 144.24 86.51) (width 0.2) (layer "F.Cu") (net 2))
 (segment (start 148.865 77.195) (end 147.828 78.232) (width 0.2) (layer "F.Cu") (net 3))
 (segment (start 147.828 78.232) (end 147.828 79.756) (width 0.2) (layer "F.Cu") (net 3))
 (segment (start 151 77.195) (end 148.865 77.195) (width 0.2) (layer "F.Cu") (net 3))
 (segment (start 147.32 80.264) (end 147.32 81.534) (width 0.2) (layer "F.Cu") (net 3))
 (segment (start 147.32 81.534) (end 147.325 81.539) (width 0.2) (layer "F.Cu") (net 3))
 (segment (start 147.325 81.539) (end 147.325 86) (width 0.2) (layer "F.Cu") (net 3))
 (segment (start 147.828 79.756) (end 147.32 80.264) (width 0.2) (layer "F.Cu") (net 3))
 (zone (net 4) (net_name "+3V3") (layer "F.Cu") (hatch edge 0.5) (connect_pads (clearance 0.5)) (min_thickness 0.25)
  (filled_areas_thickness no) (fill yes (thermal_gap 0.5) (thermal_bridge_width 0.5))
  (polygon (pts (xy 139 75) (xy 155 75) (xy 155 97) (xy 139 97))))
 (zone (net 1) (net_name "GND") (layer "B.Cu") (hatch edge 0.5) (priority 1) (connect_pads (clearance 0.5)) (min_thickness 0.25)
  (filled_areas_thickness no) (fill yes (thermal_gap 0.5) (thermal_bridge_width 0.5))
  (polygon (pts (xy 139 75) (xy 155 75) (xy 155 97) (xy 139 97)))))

